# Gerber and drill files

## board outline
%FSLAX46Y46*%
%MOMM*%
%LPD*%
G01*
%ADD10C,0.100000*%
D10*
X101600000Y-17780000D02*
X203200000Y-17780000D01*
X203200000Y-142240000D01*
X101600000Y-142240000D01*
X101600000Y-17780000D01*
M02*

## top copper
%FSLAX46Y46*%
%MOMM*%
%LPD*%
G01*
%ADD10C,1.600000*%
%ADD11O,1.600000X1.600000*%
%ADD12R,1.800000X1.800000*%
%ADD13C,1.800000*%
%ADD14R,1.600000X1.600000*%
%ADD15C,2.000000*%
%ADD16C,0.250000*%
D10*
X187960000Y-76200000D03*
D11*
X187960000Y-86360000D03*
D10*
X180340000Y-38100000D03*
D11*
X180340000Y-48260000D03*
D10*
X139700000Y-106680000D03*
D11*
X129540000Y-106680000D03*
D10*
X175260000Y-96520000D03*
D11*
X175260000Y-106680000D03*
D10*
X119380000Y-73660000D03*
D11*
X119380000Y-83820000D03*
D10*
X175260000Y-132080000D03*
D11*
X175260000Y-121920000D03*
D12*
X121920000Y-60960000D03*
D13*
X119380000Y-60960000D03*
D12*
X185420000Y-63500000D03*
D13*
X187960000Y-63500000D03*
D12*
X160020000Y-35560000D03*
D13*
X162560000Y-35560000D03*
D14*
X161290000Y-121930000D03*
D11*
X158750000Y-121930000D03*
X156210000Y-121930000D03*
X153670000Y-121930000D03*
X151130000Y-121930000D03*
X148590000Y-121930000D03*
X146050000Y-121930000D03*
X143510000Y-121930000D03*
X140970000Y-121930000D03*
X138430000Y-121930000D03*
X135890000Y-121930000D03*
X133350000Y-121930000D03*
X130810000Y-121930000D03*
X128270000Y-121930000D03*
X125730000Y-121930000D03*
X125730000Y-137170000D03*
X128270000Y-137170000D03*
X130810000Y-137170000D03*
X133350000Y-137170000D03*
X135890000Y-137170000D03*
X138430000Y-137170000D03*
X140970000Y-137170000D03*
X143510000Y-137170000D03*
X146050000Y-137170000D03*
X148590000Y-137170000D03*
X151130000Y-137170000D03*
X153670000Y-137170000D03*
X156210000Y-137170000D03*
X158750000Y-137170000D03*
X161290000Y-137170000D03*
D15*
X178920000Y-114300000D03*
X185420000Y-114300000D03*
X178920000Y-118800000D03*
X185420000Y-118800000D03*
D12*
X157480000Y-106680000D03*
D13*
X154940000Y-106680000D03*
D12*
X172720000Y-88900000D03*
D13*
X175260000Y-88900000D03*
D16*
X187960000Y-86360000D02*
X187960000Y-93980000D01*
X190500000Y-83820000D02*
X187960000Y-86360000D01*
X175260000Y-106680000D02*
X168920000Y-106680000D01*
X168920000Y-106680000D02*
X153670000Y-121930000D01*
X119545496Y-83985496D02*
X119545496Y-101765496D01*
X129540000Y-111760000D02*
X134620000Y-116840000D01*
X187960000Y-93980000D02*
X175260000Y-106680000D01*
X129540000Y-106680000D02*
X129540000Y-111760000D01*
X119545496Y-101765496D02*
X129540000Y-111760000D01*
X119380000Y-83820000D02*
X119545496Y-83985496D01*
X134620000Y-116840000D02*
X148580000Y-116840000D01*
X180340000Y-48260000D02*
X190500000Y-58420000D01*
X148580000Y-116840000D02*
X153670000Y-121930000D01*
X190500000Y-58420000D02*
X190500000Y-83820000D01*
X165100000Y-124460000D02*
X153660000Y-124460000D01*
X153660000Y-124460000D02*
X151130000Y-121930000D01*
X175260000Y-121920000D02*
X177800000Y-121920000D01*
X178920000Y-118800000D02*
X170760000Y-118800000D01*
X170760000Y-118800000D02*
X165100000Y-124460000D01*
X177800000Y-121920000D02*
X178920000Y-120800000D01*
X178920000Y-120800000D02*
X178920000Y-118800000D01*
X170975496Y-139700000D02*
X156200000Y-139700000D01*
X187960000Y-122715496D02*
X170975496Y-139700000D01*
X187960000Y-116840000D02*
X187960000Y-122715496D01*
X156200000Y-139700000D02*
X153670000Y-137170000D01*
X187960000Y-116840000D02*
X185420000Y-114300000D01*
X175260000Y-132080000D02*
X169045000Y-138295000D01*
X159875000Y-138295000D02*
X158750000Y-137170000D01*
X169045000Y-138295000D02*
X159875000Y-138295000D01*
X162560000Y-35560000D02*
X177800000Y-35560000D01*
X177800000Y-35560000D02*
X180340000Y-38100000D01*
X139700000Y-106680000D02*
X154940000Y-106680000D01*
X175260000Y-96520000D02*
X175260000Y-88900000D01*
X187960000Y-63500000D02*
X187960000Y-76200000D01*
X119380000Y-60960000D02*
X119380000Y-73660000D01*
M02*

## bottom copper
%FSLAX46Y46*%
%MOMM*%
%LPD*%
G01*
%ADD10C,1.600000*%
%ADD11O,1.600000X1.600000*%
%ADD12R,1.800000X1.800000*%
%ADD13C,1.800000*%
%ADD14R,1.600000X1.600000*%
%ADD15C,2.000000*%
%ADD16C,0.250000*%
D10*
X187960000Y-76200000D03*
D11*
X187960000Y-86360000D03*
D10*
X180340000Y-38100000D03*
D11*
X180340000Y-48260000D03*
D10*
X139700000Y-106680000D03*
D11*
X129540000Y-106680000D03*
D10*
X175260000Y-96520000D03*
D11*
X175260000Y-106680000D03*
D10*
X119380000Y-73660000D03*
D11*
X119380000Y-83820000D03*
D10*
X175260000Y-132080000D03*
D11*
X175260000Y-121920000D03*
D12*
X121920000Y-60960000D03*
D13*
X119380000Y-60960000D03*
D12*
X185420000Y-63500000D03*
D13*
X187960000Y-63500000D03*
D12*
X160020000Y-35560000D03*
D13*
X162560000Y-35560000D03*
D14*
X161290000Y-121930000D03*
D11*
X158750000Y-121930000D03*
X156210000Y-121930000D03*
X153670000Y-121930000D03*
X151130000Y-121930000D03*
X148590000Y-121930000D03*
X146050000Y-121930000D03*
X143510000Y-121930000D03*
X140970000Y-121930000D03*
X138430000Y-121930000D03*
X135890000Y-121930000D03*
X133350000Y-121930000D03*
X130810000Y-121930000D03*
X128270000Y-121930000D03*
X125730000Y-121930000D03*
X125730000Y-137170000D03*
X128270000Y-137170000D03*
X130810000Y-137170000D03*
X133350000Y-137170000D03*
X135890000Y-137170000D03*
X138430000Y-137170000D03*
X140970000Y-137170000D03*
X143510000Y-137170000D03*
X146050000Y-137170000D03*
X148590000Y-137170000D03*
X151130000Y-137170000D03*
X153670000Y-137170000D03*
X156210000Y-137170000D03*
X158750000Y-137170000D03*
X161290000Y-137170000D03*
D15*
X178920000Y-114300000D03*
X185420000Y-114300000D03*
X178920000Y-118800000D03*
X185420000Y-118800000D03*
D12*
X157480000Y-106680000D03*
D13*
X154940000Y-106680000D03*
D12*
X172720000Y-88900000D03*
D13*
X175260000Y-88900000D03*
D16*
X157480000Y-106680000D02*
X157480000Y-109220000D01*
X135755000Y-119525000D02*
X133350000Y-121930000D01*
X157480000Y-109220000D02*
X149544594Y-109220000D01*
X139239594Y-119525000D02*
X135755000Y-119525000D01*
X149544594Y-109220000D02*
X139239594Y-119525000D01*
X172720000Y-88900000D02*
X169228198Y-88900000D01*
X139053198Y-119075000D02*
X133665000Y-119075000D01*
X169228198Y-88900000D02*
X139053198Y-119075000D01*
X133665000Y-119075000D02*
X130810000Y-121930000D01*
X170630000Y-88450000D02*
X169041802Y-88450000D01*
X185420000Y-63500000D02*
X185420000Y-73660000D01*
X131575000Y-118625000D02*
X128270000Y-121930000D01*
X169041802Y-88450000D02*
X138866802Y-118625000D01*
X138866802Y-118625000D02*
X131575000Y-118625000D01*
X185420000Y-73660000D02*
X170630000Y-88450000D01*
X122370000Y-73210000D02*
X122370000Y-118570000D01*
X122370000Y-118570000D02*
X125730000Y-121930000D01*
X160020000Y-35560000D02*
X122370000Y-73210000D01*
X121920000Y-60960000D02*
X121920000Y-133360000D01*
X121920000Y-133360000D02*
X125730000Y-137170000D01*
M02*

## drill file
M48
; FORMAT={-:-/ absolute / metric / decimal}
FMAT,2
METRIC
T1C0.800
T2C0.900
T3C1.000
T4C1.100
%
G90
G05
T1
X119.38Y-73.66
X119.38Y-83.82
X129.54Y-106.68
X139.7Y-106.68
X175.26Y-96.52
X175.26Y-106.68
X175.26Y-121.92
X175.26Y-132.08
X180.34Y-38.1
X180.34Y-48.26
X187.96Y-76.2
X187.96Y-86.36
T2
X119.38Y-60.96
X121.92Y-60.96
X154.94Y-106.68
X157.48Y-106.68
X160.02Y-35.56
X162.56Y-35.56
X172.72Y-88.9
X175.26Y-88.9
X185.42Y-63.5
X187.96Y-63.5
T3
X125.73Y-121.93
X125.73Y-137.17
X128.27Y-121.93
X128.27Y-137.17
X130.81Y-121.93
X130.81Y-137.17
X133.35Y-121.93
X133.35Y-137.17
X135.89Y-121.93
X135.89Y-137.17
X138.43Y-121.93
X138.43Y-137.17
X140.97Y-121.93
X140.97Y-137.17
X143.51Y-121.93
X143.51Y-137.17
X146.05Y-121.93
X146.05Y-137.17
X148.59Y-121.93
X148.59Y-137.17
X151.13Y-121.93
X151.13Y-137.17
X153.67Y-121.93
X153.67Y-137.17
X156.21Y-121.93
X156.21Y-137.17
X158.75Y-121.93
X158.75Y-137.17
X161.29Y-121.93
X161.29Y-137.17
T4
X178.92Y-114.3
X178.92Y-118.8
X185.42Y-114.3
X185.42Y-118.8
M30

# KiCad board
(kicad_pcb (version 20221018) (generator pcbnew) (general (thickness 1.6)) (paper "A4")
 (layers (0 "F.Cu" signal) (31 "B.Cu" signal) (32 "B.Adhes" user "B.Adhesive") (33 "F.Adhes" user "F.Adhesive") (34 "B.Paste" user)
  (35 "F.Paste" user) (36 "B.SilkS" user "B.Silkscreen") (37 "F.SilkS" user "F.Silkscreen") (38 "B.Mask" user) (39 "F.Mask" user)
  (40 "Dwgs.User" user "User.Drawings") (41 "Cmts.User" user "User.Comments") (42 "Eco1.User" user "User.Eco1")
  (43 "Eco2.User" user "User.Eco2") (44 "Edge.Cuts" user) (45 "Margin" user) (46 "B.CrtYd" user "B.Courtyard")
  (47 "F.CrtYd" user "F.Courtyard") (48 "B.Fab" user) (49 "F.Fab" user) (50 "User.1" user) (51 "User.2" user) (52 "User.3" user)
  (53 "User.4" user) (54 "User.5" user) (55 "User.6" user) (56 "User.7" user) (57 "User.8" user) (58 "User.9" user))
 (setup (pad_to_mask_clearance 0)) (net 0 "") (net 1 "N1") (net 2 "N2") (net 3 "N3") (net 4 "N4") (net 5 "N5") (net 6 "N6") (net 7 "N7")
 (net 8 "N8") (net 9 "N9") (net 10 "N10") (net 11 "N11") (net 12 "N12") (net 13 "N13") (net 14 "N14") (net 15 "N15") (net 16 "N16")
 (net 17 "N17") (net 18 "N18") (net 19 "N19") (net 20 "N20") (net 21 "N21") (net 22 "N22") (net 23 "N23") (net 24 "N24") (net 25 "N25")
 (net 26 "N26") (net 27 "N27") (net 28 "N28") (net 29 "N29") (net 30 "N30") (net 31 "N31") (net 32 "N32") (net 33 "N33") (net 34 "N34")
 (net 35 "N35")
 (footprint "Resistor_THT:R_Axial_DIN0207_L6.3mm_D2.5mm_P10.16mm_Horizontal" (layer "F.Cu") (at 187.96 76.2 -90)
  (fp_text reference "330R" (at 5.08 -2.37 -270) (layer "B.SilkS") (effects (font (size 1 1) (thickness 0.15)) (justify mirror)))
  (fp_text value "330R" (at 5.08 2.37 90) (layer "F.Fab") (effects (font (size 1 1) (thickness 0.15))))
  (pad "1" thru_hole circle (at 0 0 270) (size 1.6 1.6) (drill 0.8) (layers "*.Cu" "*.Mask") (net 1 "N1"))
  (pad "2" thru_hole oval (at 10.16 0 270) (size 1.6 1.6) (drill 0.8) (layers "*.Cu" "*.Mask") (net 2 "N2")))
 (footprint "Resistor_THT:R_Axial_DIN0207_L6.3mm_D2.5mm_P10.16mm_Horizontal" (layer "F.Cu") (at 180.34 38.1 -90)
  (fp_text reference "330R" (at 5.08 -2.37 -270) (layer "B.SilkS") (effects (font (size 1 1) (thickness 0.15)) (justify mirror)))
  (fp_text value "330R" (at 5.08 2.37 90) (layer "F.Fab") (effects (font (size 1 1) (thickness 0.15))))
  (pad "1" thru_hole circle (at 0 0 270) (size 1.6 1.6) (drill 0.8) (layers "*.Cu" "*.Mask") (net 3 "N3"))
  (pad "2" thru_hole oval (at 10.16 0 270) (size 1.6 1.6) (drill 0.8) (layers "*.Cu" "*.Mask") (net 2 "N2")))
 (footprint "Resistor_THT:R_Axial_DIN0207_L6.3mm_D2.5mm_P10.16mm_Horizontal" (layer "F.Cu") (at 139.7 106.68 180)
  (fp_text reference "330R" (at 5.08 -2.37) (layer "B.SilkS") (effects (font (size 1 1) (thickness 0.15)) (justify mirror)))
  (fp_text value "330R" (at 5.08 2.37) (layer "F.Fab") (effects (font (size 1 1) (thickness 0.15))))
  (pad "1" thru_hole circle (at 0 0 180) (size 1.6 1.6) (drill 0.8) (layers "*.Cu" "*.Mask") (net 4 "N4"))
  (pad "2" thru_hole oval (at 10.16 0 180) (size 1.6 1.6) (drill 0.8) (layers "*.Cu" "*.Mask") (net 2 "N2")))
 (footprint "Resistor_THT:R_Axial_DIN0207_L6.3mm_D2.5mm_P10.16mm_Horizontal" (layer "F.Cu") (at 175.26 96.52 -90)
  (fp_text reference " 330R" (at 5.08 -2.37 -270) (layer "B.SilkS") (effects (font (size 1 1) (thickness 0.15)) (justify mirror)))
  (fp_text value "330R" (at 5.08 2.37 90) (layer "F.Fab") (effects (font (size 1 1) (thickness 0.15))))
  (pad "1" thru_hole circle (at 0 0 270) (size 1.6 1.6) (drill 0.8) (layers "*.Cu" "*.Mask") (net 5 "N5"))
  (pad "2" thru_hole oval (at 10.16 0 270) (size 1.6 1.6) (drill 0.8) (layers "*.Cu" "*.Mask") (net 2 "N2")))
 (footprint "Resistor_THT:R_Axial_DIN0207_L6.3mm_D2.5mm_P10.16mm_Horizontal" (layer "F.Cu") (at 119.38 73.66 -90)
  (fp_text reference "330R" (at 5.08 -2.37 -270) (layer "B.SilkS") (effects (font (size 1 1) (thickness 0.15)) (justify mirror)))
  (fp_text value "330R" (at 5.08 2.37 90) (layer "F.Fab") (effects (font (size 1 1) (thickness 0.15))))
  (pad "1" thru_hole circle (at 0 0 270) (size 1.6 1.6) (drill 0.8) (layers "*.Cu" "*.Mask") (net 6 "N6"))
  (pad "2" thru_hole oval (at 10.16 0 270) (size 1.6 1.6) (drill 0.8) (layers "*.Cu" "*.Mask") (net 2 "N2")))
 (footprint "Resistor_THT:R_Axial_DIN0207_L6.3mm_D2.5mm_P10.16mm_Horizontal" (layer "F.Cu") (at 175.26 132.08 90)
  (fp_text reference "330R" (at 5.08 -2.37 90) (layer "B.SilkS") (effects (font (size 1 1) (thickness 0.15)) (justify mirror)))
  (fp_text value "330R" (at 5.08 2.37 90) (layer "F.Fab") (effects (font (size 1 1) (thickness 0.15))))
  (pad "1" thru_hole circle (at 0 0 90) (size 1.6 1.6) (drill 0.8) (layers "*.Cu" "*.Mask") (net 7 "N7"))
  (pad "2" thru_hole oval (at 10.16 0 90) (size 1.6 1.6) (drill 0.8) (layers "*.Cu" "*.Mask") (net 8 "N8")))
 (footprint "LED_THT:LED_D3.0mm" (layer "F.Cu") (at 121.92 60.96 180)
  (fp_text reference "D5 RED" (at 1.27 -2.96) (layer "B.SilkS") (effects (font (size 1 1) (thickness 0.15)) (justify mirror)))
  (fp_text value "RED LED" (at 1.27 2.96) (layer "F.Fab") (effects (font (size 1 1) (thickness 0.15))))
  (pad "1" thru_hole rect (at 0 0 180) (size 1.8 1.8) (drill 0.9) (layers "*.Cu" "*.Mask") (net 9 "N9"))
  (pad "2" thru_hole circle (at 2.54 0 180) (size 1.8 1.8) (drill 0.9) (layers "*.Cu" "*.Mask") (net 6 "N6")))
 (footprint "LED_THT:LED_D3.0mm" (layer "F.Cu") (at 185.42 63.5)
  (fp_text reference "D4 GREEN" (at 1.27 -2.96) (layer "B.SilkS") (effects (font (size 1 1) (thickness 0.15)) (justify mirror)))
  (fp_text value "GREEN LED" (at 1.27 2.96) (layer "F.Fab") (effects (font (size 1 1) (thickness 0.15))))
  (pad "1" thru_hole rect (at 0 0) (size 1.8 1.8) (drill 0.9) (layers "*.Cu" "*.Mask") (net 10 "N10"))
  (pad "2" thru_hole circle (at 2.54 0) (size 1.8 1.8) (drill 0.9) (layers "*.Cu" "*.Mask") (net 1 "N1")))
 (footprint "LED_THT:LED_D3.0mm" (layer "F.Cu") (at 160.02 35.56)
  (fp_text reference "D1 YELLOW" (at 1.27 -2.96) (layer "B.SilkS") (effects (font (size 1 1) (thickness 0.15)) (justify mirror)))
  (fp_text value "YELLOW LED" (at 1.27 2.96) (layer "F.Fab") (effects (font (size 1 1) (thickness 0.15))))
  (pad "1" thru_hole rect (at 0 0) (size 1.8 1.8) (drill 0.9) (layers "*.Cu" "*.Mask") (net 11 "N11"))
  (pad "2" thru_hole circle (at 2.54 0) (size 1.8 1.8) (drill 0.9) (layers "*.Cu" "*.Mask") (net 3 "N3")))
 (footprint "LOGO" (layer "F.Cu") (at 152.4 68.58)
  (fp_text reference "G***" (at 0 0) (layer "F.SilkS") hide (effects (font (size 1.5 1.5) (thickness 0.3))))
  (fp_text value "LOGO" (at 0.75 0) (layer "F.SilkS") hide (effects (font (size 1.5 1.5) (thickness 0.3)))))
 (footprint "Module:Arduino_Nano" (layer "F.Cu") (at 161.29 121.93 -90)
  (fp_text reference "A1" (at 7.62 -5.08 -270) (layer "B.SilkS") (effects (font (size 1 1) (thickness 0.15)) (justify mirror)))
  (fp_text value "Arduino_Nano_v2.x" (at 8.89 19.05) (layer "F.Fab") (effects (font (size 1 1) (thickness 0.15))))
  (pad "1" thru_hole rect (at 0 0 270) (size 1.6 1.6) (drill 1) (layers "*.Cu" "*.Mask") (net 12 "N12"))
  (pad "2" thru_hole oval (at 0 2.54 270) (size 1.6 1.6) (drill 1) (layers "*.Cu" "*.Mask") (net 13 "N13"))
  (pad "3" thru_hole oval (at 0 5.08 270) (size 1.6 1.6) (drill 1) (layers "*.Cu" "*.Mask") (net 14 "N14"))
  (pad "4" thru_hole oval (at 0 7.62 270) (size 1.6 1.6) (drill 1) (layers "*.Cu" "*.Mask") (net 2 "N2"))
  (pad "5" thru_hole oval (at 0 10.16 270) (size 1.6 1.6) (drill 1) (layers "*.Cu" "*.Mask") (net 8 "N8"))
  (pad "6" thru_hole oval (at 0 12.7 270) (size 1.6 1.6) (drill 1) (layers "*.Cu" "*.Mask") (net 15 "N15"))
  (pad "7" thru_hole oval (at 0 15.24 270) (size 1.6 1.6) (drill 1) (layers "*.Cu" "*.Mask") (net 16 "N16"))
  (pad "8" thru_hole oval (at 0 17.78 270) (size 1.6 1.6) (drill 1) (layers "*.Cu" "*.Mask") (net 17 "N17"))
  (pad "9" thru_hole oval (at 0 20.32 270) (size 1.6 1.6) (drill 1) (layers "*.Cu" "*.Mask") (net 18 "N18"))
  (pad "10" thru_hole oval (at 0 22.86 270) (size 1.6 1.6) (drill 1) (layers "*.Cu" "*.Mask") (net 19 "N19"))
  (pad "11" thru_hole oval (at 0 25.4 270) (size 1.6 1.6) (drill 1) (layers "*.Cu" "*.Mask") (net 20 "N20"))
  (pad "12" thru_hole oval (at 0 27.94 270) (size 1.6 1.6) (drill 1) (layers "*.Cu" "*.Mask") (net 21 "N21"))
  (pad "13" thru_hole oval (at 0 30.48 270) (size 1.6 1.6) (drill 1) (layers "*.Cu" "*.Mask") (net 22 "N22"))
  (pad "14" thru_hole oval (at 0 33.02 270) (size 1.6 1.6) (drill 1) (layers "*.Cu" "*.Mask") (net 10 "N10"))
  (pad "15" thru_hole oval (at 0 35.56 270) (size 1.6 1.6) (drill 1) (layers "*.Cu" "*.Mask") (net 11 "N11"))
  (pad "16" thru_hole oval (at 15.24 35.56 270) (size 1.6 1.6) (drill 1) (layers "*.Cu" "*.Mask") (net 9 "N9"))
  (pad "17" thru_hole oval (at 15.24 33.02 270) (size 1.6 1.6) (drill 1) (layers "*.Cu" "*.Mask") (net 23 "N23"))
  (pad "18" thru_hole oval (at 15.24 30.48 270) (size 1.6 1.6) (drill 1) (layers "*.Cu" "*.Mask") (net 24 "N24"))
  (pad "19" thru_hole oval (at 15.24 27.94 270) (size 1.6 1.6) (drill 1) (layers "*.Cu" "*.Mask") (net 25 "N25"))
  (pad "20" thru_hole oval (at 15.24 25.4 270) (size 1.6 1.6) (drill 1) (layers "*.Cu" "*.Mask") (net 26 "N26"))
  (pad "21" thru_hole oval (at 15.24 22.86 270) (size 1.6 1.6) (drill 1) (layers "*.Cu" "*.Mask") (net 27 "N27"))
  (pad "22" thru_hole oval (at 15.24 20.32 270) (size 1.6 1.6) (drill 1) (layers "*.Cu" "*.Mask") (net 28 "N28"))
  (pad "23" thru_hole oval (at 15.24 17.78 270) (size 1.6 1.6) (drill 1) (layers "*.Cu" "*.Mask") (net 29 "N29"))
  (pad "24" thru_hole oval (at 15.24 15.24 270) (size 1.6 1.6) (drill 1) (layers "*.Cu" "*.Mask") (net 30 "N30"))
  (pad "25" thru_hole oval (at 15.24 12.7 270) (size 1.6 1.6) (drill 1) (layers "*.Cu" "*.Mask") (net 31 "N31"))
  (pad "26" thru_hole oval (at 15.24 10.16 270) (size 1.6 1.6) (drill 1) (layers "*.Cu" "*.Mask") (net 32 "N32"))
  (pad "27" thru_hole oval (at 15.24 7.62 270) (size 1.6 1.6) (drill 1) (layers "*.Cu" "*.Mask") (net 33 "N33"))
  (pad "28" thru_hole oval (at 15.24 5.08 270) (size 1.6 1.6) (drill 1) (layers "*.Cu" "*.Mask") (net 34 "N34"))
  (pad "29" thru_hole oval (at 15.24 2.54 270) (size 1.6 1.6) (drill 1) (layers "*.Cu" "*.Mask") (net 7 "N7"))
  (pad "30" thru_hole oval (at 15.24 0 270) (size 1.6 1.6) (drill 1) (layers "*.Cu" "*.Mask") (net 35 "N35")))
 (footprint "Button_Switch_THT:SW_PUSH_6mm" (layer "F.Cu") (at 178.92 114.3)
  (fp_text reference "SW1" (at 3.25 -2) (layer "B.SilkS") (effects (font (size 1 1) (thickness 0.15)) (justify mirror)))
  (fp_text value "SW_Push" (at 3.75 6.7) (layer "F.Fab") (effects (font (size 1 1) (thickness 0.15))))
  (pad "1" thru_hole circle (at 0 0 90) (size 2 2) (drill 1.1) (layers "*.Cu" "*.Mask") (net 33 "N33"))
  (pad "1" thru_hole circle (at 6.5 0 90) (size 2 2) (drill 1.1) (layers "*.Cu" "*.Mask") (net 33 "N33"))
  (pad "2" thru_hole circle (at 0 4.5 90) (size 2 2) (drill 1.1) (layers "*.Cu" "*.Mask") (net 8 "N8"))
  (pad "2" thru_hole circle (at 6.5 4.5 90) (size 2 2) (drill 1.1) (layers "*.Cu" "*.Mask") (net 8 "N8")))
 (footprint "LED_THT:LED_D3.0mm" (layer "F.Cu") (at 157.48 106.68 180)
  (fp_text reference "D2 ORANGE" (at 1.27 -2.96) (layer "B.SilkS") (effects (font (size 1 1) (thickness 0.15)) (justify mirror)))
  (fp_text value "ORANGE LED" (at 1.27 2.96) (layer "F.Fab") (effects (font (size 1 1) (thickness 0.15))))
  (pad "1" thru_hole rect (at 0 0 180) (size 1.8 1.8) (drill 0.9) (layers "*.Cu" "*.Mask") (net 21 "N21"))
  (pad "2" thru_hole circle (at 2.54 0 180) (size 1.8 1.8) (drill 0.9) (layers "*.Cu" "*.Mask") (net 4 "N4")))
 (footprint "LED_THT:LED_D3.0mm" (layer "F.Cu") (at 172.72 88.9)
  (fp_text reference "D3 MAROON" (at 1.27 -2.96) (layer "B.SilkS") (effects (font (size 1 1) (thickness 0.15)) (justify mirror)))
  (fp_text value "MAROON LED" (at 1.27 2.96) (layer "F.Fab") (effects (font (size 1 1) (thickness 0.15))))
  (pad "1" thru_hole rect (at 0 0) (size 1.8 1.8) (drill 0.9) (layers "*.Cu" "*.Mask") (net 22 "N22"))
  (pad "2" thru_hole circle (at 2.54 0) (size 1.8 1.8) (drill 0.9) (layers "*.Cu" "*.Mask") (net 5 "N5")))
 (gr_rect (start 101.6 17.78) (end 203.2 142.24) (stroke (width 0.1) (type default)) (fill none) (layer "Edge.Cuts"))
 (segment (start 187.96 86.36) (end 187.96 93.98) (width 0.25) (layer "F.Cu") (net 2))
 (segment (start 190.5 83.82) (end 187.96 86.36) (width 0.25) (layer "F.Cu") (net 2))
 (segment (start 175.26 106.68) (end 168.92 106.68) (width 0.25) (layer "F.Cu") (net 2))
 (segment (start 168.92 106.68) (end 153.67 121.93) (width 0.25) (layer "F.Cu") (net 2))
 (segment (start 119.545496 83.985496) (end 119.545496 101.765496) (width 0.25) (layer "F.Cu") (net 2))
 (segment (start 129.54 111.76) (end 134.62 116.84) (width 0.25) (layer "F.Cu") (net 2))
 (segment (start 187.96 93.98) (end 175.26 106.68) (width 0.25) (layer "F.Cu") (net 2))
 (segment (start 129.54 106.68) (end 129.54 111.76) (width 0.25) (layer "F.Cu") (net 2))
 (segment (start 119.545496 101.765496) (end 129.54 111.76) (width 0.25) (layer "F.Cu") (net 2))
 (segment (start 119.38 83.82) (end 119.545496 83.985496) (width 0.25) (layer "F.Cu") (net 2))
 (segment (start 134.62 116.84) (end 148.58 116.84) (width 0.25) (layer "F.Cu") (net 2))
 (segment (start 180.34 48.26) (end 190.5 58.42) (width 0.25) (layer "F.Cu") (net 2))
 (segment (start 148.58 116.84) (end 153.67 121.93) (width 0.25) (layer "F.Cu") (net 2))
 (segment (start 190.5 58.42) (end 190.5 83.82) (width 0.25) (layer "F.Cu") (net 2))
 (segment (start 165.1 124.46) (end 153.66 124.46) (width 0.25) (layer "F.Cu") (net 8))
 (segment (start 153.66 124.46) (end 151.13 121.93) (width 0.25) (layer "F.Cu") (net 8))
 (segment (start 175.26 121.92) (end 177.8 121.92) (width 0.25) (layer "F.Cu") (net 8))
 (segment (start 178.92 118.8) (end 170.76 118.8) (width 0.25) (layer "F.Cu") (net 8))
 (segment (start 170.76 118.8) (end 165.1 124.46) (width 0.25) (layer "F.Cu") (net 8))
 (segment (start 177.8 121.92) (end 178.92 120.8) (width 0.25) (layer "F.Cu") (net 8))
 (segment (start 178.92 120.8) (end 178.92 118.8) (width 0.25) (layer "F.Cu") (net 8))
 (segment (start 157.48 106.68) (end 157.48 109.22) (width 0.25) (layer "B.Cu") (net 21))
 (segment (start 135.755 119.525) (end 133.35 121.93) (width 0.25) (layer "B.Cu") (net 21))
 (segment (start 157.48 109.22) (end 149.544594 109.22) (width 0.25) (layer "B.Cu") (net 21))
 (segment (start 139.239594 119.525) (end 135.755 119.525) (width 0.25) (layer "B.Cu") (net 21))
 (segment (start 149.544594 109.22) (end 139.239594 119.525) (width 0.25) (layer "B.Cu") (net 21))
 (segment (start 172.72 88.9) (end 169.228198 88.9) (width 0.25) (layer "B.Cu") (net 22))
 (segment (start 139.053198 119.075) (end 133.665 119.075) (width 0.25) (layer "B.Cu") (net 22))
 (segment (start 169.228198 88.9) (end 139.053198 119.075) (width 0.25) (layer "B.Cu") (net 22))
 (segment (start 133.665 119.075) (end 130.81 121.93) (width 0.25) (layer "B.Cu") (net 22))
 (segment (start 170.63 88.45) (end 169.041802 88.45) (width 0.25) (layer "B.Cu") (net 10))
 (segment (start 185.42 63.5) (end 185.42 73.66) (width 0.25) (layer "B.Cu") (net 10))
 (segment (start 131.575 118.625) (end 128.27 121.93) (width 0.25) (layer "B.Cu") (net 10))
 (segment (start 169.041802 88.45) (end 138.866802 118.625) (width 0.25) (layer "B.Cu") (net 10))
 (segment (start 138.866802 118.625) (end 131.575 118.625) (width 0.25) (layer "B.Cu") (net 10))
 (segment (start 185.42 73.66) (end 170.63 88.45) (width 0.25) (layer "B.Cu") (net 10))
 (segment (start 122.37 73.21) (end 122.37 118.57) (width 0.25) (layer "B.Cu") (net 11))
 (segment (start 122.37 118.57) (end 125.73 121.93) (width 0.25) (layer "B.Cu") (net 11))
 (segment (start 160.02 35.56) (end 122.37 73.21) (width 0.25) (layer "B.Cu") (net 11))
 (segment (start 121.92 60.96) (end 121.92 133.36) (width 0.25) (layer "B.Cu") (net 9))
 (segment (start 121.92 133.36) (end 125.73 137.17) (width 0.25) (layer "B.Cu") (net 9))
 (segment (start 170.975496 139.7) (end 156.2 139.7) (width 0.25) (layer "F.Cu") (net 33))
 (segment (start 187.96 122.715496) (end 170.975496 139.7) (width 0.25) (layer "F.Cu") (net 33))
 (segment (start 187.96 116.84) (end 187.96 122.715496) (width 0.25) (layer "F.Cu") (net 33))
 (segment (start 156.2 139.7) (end 153.67 137.17) (width 0.25) (layer "F.Cu") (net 33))
 (segment (start 187.96 116.84) (end 185.42 114.3) (width 0.25) (layer "F.Cu") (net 33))
 (segment (start 175.26 132.08) (end 169.045 138.295) (width 0.25) (layer "F.Cu") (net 7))
 (segment (start 159.875 138.295) (end 158.75 137.17) (width 0.25) (layer "F.Cu") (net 7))
 (segment (start 169.045 138.295) (end 159.875 138.295) (width 0.25) (layer "F.Cu") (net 7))
 (segment (start 162.56 35.56) (end 177.8 35.56) (width 0.25) (layer "F.Cu") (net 3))
 (segment (start 177.8 35.56) (end 180.34 38.1) (width 0.25) (layer "F.Cu") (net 3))
 (segment (start 139.7 106.68) (end 154.94 106.68) (width 0.25) (layer "F.Cu") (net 4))
 (segment (start 175.26 96.52) (end 175.26 88.9) (width 0.25) (layer "F.Cu") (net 5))
 (segment (start 187.96 63.5) (end 187.96 76.2) (width 0.25) (layer "F.Cu") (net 1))
 (segment (start 119.38 60.96) (end 119.38 73.66) (width 0.25) (layer "F.Cu") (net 6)))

